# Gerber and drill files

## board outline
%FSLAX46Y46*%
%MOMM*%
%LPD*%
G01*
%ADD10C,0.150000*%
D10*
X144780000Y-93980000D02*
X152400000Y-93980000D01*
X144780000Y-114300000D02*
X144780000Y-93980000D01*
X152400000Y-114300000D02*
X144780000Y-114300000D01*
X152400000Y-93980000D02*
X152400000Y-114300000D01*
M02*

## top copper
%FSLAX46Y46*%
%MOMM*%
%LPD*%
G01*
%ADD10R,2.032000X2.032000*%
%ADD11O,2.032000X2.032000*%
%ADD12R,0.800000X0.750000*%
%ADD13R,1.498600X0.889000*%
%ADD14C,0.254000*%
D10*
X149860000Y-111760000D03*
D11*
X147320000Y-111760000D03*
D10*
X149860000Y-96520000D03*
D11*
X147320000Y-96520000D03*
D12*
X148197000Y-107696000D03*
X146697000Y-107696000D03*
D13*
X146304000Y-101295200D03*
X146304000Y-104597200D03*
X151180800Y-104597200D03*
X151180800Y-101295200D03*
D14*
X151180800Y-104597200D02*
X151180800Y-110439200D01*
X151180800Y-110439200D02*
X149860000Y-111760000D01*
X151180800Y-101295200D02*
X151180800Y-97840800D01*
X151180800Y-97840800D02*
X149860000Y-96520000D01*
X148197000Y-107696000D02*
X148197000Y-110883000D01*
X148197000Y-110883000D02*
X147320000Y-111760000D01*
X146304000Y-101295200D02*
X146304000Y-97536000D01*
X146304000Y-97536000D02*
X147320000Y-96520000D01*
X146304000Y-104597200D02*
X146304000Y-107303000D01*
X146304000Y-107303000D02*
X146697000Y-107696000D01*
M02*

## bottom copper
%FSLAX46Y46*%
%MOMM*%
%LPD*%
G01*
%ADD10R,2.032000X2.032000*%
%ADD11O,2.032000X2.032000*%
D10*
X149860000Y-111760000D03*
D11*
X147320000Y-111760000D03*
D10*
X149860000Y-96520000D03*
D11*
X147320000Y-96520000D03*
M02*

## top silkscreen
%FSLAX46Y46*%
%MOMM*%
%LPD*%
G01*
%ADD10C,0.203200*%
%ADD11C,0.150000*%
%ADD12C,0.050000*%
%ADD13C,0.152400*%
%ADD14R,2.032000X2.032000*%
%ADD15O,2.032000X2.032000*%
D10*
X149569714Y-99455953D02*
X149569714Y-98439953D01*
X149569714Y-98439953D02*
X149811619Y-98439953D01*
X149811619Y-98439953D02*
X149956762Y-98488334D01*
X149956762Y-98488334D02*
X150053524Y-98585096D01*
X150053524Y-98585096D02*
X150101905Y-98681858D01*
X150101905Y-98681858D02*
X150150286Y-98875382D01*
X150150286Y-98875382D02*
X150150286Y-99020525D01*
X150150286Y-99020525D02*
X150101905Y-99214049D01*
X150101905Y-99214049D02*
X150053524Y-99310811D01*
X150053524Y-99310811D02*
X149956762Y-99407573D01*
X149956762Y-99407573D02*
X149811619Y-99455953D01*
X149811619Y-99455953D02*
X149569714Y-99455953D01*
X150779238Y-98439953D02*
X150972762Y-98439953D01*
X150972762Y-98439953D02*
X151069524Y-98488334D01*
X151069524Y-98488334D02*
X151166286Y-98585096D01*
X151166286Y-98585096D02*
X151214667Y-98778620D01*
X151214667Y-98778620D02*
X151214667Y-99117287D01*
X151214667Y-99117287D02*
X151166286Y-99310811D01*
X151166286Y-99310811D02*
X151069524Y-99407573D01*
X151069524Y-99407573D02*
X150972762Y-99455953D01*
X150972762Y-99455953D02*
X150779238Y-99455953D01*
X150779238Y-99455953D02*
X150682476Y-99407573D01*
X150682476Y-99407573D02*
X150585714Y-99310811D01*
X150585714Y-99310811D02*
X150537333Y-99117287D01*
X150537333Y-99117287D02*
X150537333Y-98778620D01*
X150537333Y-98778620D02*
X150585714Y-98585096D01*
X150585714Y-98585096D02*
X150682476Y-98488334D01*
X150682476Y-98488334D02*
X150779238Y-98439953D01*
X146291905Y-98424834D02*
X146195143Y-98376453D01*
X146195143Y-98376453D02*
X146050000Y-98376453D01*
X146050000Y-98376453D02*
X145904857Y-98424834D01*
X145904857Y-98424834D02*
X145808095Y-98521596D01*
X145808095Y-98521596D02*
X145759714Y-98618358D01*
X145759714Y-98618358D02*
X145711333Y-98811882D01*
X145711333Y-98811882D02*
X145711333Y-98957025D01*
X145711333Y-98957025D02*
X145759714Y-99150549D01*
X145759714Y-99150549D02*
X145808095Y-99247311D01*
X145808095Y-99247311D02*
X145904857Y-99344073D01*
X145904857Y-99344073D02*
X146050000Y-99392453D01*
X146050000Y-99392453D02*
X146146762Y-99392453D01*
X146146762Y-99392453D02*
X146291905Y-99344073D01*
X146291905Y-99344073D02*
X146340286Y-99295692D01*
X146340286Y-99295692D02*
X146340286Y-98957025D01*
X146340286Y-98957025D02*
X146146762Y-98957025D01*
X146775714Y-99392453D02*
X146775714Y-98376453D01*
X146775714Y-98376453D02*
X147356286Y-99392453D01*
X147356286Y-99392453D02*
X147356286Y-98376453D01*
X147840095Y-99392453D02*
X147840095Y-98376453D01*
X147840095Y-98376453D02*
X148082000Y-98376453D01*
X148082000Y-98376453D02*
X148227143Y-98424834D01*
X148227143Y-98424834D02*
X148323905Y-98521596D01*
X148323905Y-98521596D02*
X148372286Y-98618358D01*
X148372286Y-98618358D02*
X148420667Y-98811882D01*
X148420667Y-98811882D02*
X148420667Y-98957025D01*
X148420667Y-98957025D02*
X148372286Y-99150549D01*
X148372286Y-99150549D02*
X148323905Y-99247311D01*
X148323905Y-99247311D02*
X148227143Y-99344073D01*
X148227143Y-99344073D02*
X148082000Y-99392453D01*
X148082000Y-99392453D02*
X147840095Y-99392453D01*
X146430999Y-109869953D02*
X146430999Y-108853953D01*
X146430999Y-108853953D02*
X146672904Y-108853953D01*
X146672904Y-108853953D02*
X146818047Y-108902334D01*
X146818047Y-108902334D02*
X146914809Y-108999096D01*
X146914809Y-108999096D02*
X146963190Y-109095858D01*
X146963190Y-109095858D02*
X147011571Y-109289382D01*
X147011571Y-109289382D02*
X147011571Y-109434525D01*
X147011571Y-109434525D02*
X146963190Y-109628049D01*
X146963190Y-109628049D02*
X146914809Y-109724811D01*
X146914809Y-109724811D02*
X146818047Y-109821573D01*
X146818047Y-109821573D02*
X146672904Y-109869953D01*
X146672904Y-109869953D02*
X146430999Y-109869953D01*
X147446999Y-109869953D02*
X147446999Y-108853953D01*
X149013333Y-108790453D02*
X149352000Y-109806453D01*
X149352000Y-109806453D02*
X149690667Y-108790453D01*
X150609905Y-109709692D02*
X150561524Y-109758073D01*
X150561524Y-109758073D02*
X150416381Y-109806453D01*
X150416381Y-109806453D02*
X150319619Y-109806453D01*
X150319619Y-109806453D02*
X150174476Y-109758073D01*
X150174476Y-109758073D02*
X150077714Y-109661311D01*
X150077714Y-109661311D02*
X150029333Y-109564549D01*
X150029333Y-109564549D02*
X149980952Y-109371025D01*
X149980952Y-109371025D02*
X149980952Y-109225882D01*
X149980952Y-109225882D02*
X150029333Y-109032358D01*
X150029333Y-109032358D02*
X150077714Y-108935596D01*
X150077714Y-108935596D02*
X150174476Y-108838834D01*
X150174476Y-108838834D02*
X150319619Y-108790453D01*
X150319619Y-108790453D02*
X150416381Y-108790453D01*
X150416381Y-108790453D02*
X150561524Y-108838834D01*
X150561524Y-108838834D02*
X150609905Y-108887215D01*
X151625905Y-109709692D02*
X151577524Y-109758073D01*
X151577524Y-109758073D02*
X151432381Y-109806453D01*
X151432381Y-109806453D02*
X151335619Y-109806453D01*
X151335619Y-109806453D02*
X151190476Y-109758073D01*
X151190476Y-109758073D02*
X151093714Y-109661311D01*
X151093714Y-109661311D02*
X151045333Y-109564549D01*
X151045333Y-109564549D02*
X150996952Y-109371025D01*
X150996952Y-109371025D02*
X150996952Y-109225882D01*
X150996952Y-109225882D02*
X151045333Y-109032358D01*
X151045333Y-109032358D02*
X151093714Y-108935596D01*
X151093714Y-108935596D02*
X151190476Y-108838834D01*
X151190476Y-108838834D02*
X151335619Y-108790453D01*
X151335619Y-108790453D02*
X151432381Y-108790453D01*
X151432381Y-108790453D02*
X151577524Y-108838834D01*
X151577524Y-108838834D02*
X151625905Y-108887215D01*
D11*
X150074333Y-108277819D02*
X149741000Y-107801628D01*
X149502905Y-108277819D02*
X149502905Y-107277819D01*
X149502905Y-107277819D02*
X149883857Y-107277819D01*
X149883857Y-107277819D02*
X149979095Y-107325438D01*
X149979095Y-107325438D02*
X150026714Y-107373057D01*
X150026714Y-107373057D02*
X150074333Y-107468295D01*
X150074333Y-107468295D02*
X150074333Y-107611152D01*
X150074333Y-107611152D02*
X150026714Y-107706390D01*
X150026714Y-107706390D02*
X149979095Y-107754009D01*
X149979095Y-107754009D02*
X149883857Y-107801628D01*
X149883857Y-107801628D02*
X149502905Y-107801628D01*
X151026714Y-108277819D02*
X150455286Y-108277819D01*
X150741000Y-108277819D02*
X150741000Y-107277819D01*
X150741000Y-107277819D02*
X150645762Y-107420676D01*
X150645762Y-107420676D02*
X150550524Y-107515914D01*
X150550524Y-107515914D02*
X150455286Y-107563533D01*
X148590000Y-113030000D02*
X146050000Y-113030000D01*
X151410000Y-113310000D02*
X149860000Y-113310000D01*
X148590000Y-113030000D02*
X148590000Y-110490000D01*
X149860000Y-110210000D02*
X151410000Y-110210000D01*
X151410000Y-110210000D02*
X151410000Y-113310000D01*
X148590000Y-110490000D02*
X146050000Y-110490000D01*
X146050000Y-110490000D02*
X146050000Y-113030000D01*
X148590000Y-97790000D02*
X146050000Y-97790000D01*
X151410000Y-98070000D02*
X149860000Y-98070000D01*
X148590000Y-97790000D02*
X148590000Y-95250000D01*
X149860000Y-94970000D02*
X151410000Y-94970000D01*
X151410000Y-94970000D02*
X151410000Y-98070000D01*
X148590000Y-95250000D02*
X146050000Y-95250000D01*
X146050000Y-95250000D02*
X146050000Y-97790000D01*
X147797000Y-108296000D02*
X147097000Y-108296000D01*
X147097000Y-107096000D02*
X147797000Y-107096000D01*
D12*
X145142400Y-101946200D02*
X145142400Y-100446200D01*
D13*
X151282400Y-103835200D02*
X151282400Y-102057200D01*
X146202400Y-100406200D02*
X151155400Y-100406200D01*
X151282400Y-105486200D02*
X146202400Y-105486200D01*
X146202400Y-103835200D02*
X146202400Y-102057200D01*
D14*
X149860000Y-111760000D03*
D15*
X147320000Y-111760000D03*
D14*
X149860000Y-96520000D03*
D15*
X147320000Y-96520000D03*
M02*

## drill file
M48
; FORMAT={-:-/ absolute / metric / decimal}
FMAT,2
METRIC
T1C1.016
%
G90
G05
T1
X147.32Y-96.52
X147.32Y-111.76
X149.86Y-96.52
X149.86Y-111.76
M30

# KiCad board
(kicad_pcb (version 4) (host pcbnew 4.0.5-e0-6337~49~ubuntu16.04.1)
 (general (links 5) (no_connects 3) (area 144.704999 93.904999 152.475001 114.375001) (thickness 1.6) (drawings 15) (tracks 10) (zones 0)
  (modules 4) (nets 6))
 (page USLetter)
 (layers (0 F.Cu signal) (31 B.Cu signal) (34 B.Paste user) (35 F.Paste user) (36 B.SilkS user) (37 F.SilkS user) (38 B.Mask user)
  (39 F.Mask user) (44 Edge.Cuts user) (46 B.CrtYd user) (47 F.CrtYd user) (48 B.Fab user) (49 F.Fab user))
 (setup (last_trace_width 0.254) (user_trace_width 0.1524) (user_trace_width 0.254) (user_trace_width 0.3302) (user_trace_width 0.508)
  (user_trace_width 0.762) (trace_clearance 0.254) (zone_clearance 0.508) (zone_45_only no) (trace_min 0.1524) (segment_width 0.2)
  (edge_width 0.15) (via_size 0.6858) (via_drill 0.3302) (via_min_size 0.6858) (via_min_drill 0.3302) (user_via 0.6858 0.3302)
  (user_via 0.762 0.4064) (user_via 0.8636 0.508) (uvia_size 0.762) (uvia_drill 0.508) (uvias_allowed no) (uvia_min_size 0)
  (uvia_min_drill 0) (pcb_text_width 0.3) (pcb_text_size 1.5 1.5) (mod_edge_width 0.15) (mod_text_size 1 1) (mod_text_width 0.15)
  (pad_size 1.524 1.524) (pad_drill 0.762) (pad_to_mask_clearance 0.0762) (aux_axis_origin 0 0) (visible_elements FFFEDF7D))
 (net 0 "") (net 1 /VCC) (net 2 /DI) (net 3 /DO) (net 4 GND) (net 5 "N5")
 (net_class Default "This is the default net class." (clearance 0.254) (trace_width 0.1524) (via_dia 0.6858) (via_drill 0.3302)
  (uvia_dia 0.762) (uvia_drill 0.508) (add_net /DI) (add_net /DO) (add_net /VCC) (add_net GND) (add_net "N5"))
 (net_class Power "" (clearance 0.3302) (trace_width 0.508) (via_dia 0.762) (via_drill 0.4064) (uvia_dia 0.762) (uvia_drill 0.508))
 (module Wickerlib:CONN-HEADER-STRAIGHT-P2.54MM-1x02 (layer F.Cu) (at 149.86 111.76 270)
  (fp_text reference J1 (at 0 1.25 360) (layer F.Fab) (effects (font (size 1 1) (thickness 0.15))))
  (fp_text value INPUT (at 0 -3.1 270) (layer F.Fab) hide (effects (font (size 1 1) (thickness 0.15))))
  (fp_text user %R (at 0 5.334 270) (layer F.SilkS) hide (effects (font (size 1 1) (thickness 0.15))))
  (fp_line (start 1.27 1.27) (end 1.27 3.81) (layer F.SilkS) (width 0.15))
  (fp_line (start 1.55 -1.55) (end 1.55 0) (layer F.SilkS) (width 0.15))
  (fp_line (start 1.27 1.27) (end -1.27 1.27) (layer F.SilkS) (width 0.15))
  (fp_line (start -1.55 0) (end -1.55 -1.55) (layer F.SilkS) (width 0.15))
  (fp_line (start -1.55 -1.55) (end 1.55 -1.55) (layer F.SilkS) (width 0.15))
  (fp_line (start -1.27 1.27) (end -1.27 3.81) (layer F.SilkS) (width 0.15))
  (fp_line (start -1.27 3.81) (end 1.27 3.81) (layer F.SilkS) (width 0.15))
  (pad 1 thru_hole rect (at 0 0 270) (size 2.032 2.032) (drill 1.016) (layers *.Cu *.Mask F.SilkS) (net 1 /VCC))
  (pad 2 thru_hole oval (at 0 2.54 270) (size 2.032 2.032) (drill 1.016) (layers *.Cu *.Mask F.SilkS) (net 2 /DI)))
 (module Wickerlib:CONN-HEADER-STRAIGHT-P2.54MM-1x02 (layer F.Cu) (at 149.86 96.52 270)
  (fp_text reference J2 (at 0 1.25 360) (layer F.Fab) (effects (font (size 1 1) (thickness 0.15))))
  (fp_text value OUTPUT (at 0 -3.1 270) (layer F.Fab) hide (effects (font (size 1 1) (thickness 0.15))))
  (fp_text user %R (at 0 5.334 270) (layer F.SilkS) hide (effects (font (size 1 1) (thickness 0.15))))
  (fp_line (start 1.27 1.27) (end 1.27 3.81) (layer F.SilkS) (width 0.15))
  (fp_line (start 1.55 -1.55) (end 1.55 0) (layer F.SilkS) (width 0.15))
  (fp_line (start 1.27 1.27) (end -1.27 1.27) (layer F.SilkS) (width 0.15))
  (fp_line (start -1.55 0) (end -1.55 -1.55) (layer F.SilkS) (width 0.15))
  (fp_line (start -1.55 -1.55) (end 1.55 -1.55) (layer F.SilkS) (width 0.15))
  (fp_line (start -1.27 1.27) (end -1.27 3.81) (layer F.SilkS) (width 0.15))
  (fp_line (start -1.27 3.81) (end 1.27 3.81) (layer F.SilkS) (width 0.15))
  (pad 1 thru_hole rect (at 0 0 270) (size 2.032 2.032) (drill 1.016) (layers *.Cu *.Mask F.SilkS) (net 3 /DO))
  (pad 2 thru_hole oval (at 0 2.54 270) (size 2.032 2.032) (drill 1.016) (layers *.Cu *.Mask F.SilkS) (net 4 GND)))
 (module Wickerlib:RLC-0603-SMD (layer F.Cu) (at 147.447 107.696 180)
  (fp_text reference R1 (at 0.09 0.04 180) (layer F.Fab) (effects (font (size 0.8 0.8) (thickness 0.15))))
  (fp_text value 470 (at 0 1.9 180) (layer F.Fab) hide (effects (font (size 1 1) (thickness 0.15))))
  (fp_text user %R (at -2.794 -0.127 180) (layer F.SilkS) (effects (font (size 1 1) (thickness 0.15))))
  (fp_line (start -0.35 -0.6) (end 0.35 -0.6) (layer F.SilkS) (width 0.15))
  (fp_line (start 0.35 0.6) (end -0.35 0.6) (layer F.SilkS) (width 0.15))
  (pad 1 smd rect (at -0.75 0 180) (size 0.8 0.75) (layers F.Cu F.Paste F.Mask) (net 2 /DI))
  (pad 2 smd rect (at 0.75 0 180) (size 0.8 0.75) (layers F.Cu F.Paste F.Mask) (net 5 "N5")))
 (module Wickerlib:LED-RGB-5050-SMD (layer F.Cu) (at 148.7424 102.9462 180)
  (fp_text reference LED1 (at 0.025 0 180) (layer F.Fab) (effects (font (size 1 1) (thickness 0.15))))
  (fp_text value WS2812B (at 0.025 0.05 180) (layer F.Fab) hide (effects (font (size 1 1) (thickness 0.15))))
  (fp_line (start 3.6 1) (end 3.6 2.5) (layer F.SilkS) (width 0.05))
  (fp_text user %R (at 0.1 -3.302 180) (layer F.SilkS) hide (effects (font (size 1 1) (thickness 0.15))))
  (fp_line (start -2.54 -0.889) (end -2.54 0.889) (layer F.SilkS) (width 0.1524))
  (fp_line (start 2.54 2.54) (end -2.413 2.54) (layer F.SilkS) (width 0.1524))
  (fp_line (start -2.54 -2.54) (end 2.54 -2.54) (layer F.SilkS) (width 0.1524))
  (fp_line (start 2.54 -0.889) (end 2.54 0.889) (layer F.SilkS) (width 0.1524))
  (pad 1 smd rect (at 2.4384 1.651 180) (size 1.4986 0.889) (layers F.Cu F.Paste F.Mask) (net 4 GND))
  (pad 2 smd rect (at 2.4384 -1.651 180) (size 1.4986 0.889) (layers F.Cu F.Paste F.Mask) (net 5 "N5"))
  (pad 3 smd rect (at -2.4384 -1.651 180) (size 1.4986 0.889) (layers F.Cu F.Paste F.Mask) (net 1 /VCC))
  (pad 4 smd rect (at -2.4384 1.651 180) (size 1.4986 0.889) (layers F.Cu F.Paste F.Mask) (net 3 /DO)))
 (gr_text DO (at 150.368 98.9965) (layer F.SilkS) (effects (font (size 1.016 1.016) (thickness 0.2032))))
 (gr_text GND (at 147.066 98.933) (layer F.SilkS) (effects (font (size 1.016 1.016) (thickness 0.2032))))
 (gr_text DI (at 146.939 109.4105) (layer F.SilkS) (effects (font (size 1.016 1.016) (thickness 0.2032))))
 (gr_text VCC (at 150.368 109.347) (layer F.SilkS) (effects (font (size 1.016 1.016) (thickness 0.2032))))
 (gr_line (start 144.78 93.98) (end 152.4 93.98) (layer Edge.Cuts) (width 0.15))
 (gr_line (start 144.78 114.3) (end 144.78 93.98) (layer Edge.Cuts) (width 0.15))
 (gr_line (start 152.4 114.3) (end 144.78 114.3) (layer Edge.Cuts) (width 0.15))
 (gr_line (start 152.4 93.98) (end 152.4 114.3) (layer Edge.Cuts) (width 0.15))
 (segment (start 151.1808 104.5972) (end 151.1808 110.4392) (width 0.254) (layer F.Cu) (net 1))
 (segment (start 151.1808 110.4392) (end 149.86 111.76) (width 0.254) (layer F.Cu) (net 1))
 (segment (start 151.1808 101.2952) (end 151.1808 97.8408) (width 0.254) (layer F.Cu) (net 3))
 (segment (start 151.1808 97.8408) (end 149.86 96.52) (width 0.254) (layer F.Cu) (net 3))
 (segment (start 148.197 107.696) (end 148.197 110.883) (width 0.254) (layer F.Cu) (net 2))
 (segment (start 148.197 110.883) (end 147.32 111.76) (width 0.254) (layer F.Cu) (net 2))
 (segment (start 146.304 101.2952) (end 146.304 97.536) (width 0.254) (layer F.Cu) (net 4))
 (segment (start 146.304 97.536) (end 147.32 96.52) (width 0.254) (layer F.Cu) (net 4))
 (segment (start 146.304 104.5972) (end 146.304 107.303) (width 0.254) (layer F.Cu) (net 5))
 (segment (start 146.304 107.303) (end 146.697 107.696) (width 0.254) (layer F.Cu) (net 5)))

